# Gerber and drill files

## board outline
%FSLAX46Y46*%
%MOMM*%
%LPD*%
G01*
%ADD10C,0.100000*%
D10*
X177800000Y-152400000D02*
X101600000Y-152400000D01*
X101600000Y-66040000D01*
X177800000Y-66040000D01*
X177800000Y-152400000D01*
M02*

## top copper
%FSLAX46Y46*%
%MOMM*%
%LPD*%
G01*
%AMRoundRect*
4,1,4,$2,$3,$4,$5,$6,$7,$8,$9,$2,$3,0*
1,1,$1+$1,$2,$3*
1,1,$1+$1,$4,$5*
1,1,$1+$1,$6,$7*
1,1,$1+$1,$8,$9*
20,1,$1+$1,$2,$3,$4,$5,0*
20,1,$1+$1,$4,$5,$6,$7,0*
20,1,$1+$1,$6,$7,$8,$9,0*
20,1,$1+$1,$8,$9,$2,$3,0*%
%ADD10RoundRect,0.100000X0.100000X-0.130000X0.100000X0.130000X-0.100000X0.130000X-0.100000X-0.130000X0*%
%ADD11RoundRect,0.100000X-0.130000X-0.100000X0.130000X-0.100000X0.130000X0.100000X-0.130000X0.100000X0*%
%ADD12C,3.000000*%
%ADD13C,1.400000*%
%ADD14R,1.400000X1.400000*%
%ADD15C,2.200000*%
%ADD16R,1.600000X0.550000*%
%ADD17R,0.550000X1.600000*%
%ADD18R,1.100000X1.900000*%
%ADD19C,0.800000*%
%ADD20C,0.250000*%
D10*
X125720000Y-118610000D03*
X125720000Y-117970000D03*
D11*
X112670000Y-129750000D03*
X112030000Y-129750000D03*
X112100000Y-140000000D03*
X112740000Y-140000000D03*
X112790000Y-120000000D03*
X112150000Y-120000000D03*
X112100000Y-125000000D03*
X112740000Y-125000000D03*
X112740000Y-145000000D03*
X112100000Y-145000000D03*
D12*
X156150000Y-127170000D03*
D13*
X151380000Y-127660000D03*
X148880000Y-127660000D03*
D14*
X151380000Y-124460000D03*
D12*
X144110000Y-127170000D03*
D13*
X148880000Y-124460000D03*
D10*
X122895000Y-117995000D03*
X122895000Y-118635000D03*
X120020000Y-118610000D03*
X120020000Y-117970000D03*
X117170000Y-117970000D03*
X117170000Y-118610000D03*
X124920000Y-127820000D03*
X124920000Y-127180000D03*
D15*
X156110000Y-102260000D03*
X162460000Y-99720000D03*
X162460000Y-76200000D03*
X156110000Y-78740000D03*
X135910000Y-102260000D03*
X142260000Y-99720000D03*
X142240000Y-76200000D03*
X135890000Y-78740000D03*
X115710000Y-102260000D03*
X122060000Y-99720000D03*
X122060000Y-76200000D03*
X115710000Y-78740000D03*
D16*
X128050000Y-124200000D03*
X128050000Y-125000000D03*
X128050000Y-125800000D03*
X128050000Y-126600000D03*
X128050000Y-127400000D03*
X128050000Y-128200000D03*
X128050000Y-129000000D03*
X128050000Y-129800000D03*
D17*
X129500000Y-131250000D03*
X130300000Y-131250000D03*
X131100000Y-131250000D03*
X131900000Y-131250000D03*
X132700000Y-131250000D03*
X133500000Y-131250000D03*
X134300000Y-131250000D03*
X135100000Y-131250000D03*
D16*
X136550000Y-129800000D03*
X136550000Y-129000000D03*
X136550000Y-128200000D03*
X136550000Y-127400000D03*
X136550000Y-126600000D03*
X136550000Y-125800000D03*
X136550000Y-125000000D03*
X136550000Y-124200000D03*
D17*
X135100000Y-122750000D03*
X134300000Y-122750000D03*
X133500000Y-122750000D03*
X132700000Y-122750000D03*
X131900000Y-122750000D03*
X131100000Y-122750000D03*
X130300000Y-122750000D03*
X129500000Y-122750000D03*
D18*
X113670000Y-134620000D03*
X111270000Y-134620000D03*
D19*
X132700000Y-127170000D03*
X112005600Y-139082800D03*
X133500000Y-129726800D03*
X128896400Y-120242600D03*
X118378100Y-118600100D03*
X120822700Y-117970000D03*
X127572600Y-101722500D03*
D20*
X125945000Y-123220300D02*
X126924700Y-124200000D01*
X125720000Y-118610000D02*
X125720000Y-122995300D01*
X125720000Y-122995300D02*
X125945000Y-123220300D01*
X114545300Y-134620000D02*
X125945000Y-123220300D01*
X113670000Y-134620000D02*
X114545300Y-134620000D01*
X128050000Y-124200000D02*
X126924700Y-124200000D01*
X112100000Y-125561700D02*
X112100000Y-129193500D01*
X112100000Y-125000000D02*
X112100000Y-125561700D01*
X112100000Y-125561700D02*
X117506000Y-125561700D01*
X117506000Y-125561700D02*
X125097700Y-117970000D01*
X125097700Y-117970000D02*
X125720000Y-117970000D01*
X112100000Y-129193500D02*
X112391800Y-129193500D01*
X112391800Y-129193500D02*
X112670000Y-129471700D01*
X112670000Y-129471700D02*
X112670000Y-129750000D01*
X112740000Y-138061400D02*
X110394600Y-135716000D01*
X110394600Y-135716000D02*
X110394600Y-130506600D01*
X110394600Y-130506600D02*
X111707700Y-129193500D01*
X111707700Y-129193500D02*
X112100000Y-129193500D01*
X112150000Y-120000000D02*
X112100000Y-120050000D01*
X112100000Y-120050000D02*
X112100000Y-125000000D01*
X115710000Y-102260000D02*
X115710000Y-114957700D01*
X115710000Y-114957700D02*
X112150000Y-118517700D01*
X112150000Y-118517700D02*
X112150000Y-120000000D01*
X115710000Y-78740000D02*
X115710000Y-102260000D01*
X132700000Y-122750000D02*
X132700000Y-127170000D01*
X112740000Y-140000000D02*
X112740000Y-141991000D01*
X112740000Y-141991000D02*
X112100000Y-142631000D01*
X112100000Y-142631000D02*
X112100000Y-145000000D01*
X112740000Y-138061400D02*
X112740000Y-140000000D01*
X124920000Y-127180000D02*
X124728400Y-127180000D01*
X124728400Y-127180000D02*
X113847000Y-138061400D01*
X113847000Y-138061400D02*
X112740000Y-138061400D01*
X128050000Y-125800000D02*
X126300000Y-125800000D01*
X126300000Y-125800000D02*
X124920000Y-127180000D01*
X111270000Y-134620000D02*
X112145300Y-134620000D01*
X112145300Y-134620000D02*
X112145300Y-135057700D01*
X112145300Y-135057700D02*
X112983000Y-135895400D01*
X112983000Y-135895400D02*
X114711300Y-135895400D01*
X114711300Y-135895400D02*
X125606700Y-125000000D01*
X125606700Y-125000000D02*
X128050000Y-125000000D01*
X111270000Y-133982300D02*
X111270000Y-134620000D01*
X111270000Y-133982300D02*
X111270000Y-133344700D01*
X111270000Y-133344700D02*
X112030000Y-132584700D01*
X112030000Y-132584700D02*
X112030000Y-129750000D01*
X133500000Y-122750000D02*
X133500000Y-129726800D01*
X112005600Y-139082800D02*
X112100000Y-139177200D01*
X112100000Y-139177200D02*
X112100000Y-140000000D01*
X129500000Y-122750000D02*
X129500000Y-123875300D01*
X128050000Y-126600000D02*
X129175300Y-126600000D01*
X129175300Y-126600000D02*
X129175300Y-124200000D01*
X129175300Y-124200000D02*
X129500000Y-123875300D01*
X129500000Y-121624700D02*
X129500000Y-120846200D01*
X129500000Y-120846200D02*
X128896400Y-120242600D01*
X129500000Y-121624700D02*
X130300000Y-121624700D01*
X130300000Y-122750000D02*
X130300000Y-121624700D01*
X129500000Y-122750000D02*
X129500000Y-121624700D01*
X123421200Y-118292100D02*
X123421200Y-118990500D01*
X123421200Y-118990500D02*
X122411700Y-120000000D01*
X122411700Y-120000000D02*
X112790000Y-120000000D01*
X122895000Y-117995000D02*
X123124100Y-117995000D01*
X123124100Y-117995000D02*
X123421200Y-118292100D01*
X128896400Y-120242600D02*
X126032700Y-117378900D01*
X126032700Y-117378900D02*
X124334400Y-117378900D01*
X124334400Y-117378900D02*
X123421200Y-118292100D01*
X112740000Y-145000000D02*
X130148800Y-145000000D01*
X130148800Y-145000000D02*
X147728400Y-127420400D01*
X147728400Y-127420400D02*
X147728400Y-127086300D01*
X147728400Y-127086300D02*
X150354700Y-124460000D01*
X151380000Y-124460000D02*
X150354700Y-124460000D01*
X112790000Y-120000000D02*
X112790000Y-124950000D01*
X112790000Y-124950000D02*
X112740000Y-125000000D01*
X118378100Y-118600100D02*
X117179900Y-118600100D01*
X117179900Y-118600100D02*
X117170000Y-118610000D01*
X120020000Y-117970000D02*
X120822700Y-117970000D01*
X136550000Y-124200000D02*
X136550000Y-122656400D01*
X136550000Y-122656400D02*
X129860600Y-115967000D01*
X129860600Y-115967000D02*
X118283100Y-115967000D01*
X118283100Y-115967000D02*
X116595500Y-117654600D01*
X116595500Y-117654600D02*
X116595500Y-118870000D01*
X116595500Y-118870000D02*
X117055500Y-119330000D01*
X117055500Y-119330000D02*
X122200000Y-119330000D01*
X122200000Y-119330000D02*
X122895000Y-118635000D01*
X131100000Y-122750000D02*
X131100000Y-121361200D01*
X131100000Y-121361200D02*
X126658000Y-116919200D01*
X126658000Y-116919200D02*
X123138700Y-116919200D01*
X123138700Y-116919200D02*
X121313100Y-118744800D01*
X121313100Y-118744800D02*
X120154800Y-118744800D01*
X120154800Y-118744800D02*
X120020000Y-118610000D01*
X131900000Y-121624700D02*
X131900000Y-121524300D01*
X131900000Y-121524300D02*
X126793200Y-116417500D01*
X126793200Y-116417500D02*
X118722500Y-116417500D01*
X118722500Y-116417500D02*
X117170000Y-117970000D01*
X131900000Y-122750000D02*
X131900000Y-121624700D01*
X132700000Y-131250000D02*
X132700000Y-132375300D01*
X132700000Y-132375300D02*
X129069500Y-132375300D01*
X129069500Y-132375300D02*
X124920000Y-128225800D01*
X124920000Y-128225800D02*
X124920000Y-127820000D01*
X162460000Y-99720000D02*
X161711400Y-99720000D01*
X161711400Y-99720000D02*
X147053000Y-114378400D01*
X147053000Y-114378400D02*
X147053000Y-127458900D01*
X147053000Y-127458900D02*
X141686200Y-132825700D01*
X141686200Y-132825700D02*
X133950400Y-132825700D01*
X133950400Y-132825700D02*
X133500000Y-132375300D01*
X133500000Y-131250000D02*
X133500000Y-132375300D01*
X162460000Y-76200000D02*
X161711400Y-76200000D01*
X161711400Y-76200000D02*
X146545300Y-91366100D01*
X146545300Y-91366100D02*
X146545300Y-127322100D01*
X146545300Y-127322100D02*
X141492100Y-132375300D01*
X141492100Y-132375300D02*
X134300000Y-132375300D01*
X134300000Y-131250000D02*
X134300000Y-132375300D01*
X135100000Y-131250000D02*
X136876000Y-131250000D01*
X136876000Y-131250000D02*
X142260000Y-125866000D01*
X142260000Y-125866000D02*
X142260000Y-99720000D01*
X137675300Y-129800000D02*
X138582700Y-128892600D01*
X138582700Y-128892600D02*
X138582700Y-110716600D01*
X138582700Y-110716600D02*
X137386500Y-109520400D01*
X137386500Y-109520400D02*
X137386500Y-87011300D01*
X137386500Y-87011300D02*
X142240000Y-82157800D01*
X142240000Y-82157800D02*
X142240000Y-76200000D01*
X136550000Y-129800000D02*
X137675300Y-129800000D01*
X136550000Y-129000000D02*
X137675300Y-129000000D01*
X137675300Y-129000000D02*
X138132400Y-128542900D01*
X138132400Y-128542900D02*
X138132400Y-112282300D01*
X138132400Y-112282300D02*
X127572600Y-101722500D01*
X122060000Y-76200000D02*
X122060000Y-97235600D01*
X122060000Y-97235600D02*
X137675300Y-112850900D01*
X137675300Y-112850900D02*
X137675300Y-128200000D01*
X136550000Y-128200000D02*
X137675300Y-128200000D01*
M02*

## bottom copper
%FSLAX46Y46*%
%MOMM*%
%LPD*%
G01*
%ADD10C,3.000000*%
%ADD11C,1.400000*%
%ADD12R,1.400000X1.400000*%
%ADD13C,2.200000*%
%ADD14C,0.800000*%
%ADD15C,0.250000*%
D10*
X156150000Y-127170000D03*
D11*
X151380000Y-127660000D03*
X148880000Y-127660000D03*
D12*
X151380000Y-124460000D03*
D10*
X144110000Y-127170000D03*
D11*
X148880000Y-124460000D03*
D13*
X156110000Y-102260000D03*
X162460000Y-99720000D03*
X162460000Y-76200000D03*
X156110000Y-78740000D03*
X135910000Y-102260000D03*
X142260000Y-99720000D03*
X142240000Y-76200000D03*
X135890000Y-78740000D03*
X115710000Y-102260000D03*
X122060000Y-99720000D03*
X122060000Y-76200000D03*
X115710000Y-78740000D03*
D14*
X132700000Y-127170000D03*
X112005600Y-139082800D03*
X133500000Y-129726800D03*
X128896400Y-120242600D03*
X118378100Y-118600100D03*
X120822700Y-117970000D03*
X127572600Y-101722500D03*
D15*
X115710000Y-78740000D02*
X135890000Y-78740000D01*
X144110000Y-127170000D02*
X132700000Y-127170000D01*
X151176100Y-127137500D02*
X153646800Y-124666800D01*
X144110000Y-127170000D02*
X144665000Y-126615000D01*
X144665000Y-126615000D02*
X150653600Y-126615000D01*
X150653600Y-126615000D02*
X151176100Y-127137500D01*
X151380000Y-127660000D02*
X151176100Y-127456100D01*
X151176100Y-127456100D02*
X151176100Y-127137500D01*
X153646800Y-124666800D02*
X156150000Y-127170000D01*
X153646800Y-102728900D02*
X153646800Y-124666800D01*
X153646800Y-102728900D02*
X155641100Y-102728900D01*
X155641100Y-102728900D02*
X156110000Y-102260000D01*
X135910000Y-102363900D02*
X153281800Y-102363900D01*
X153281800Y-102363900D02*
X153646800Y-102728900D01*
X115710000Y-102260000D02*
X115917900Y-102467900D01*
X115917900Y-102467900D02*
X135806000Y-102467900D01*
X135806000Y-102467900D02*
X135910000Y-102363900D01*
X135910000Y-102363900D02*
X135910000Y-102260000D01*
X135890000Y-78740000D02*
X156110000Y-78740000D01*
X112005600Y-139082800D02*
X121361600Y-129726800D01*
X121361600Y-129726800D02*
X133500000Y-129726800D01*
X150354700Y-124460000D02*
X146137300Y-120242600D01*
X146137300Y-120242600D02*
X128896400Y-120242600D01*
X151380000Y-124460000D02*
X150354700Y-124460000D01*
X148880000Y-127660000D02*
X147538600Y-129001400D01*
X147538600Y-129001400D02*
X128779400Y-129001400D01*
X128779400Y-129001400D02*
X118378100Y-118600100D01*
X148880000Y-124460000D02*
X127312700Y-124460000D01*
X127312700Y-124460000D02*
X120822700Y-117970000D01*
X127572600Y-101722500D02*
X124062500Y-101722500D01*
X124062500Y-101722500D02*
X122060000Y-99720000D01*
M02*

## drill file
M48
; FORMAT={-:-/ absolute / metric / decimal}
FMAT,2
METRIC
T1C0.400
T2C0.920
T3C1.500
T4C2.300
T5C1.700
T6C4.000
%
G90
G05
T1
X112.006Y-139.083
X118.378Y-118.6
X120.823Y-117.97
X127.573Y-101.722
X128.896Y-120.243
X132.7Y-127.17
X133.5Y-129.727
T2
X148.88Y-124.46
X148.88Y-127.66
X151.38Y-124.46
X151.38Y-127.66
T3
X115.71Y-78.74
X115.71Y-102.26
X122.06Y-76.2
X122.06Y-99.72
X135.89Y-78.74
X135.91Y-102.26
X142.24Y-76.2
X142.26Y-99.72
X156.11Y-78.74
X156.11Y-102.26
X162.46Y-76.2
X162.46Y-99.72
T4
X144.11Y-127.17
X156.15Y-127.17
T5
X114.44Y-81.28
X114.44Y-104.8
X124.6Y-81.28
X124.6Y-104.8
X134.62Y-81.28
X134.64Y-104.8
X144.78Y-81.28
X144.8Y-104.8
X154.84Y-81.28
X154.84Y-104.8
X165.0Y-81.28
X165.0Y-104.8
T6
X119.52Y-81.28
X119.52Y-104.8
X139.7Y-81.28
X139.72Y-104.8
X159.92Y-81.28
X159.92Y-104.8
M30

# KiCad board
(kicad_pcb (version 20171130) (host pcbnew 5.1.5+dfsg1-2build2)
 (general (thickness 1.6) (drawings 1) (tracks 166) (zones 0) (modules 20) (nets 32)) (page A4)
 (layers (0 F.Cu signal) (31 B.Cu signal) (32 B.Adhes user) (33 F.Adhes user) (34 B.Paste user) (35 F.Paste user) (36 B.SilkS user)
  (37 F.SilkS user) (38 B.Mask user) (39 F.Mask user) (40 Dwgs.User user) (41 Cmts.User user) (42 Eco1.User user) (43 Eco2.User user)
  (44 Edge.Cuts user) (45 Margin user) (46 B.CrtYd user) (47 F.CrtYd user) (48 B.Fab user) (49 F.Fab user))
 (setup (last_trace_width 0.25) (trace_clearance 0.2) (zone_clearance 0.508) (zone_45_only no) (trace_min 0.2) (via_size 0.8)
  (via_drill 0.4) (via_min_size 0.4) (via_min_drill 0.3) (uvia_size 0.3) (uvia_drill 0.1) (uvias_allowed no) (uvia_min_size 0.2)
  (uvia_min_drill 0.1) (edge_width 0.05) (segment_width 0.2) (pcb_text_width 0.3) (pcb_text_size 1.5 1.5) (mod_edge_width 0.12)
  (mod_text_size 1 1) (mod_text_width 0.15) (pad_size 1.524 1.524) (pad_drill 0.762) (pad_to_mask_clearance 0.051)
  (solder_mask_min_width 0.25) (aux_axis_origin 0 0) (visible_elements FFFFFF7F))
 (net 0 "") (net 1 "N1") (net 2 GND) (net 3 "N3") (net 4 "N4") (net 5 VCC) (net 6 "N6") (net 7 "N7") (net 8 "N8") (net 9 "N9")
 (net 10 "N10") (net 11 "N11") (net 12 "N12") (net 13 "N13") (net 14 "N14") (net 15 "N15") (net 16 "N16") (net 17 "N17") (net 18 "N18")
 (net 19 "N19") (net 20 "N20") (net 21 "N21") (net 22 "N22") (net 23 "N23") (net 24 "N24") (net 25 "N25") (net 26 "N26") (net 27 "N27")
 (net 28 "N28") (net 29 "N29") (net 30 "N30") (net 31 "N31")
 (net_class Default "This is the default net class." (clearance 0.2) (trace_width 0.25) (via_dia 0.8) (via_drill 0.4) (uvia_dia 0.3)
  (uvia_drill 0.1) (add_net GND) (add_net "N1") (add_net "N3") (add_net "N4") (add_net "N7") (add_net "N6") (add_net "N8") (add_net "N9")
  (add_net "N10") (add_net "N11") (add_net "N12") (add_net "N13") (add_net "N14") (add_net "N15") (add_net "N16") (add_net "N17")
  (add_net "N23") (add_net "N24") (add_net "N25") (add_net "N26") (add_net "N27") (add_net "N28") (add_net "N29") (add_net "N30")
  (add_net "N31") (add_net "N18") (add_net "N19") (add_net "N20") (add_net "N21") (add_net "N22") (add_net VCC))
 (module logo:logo (layer F.Cu) (at 149.86 141.5)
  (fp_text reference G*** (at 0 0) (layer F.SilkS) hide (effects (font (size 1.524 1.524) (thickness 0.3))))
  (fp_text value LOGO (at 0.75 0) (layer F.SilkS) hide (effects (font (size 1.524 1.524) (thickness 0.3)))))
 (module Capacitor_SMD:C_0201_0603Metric (layer F.Cu) (at 125.72 118.29 90)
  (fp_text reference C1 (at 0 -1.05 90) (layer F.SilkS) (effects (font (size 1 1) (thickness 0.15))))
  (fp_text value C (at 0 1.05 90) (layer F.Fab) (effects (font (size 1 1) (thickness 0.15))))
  (pad "" smd roundrect (at -0.345 0 90) (size 0.318 0.36) (layers F.Paste) (roundrect_rratio 0.25))
  (pad "" smd roundrect (at 0.345 0 90) (size 0.318 0.36) (layers F.Paste) (roundrect_rratio 0.25))
  (pad 1 smd roundrect (at -0.32 0 90) (size 0.46 0.4) (layers F.Cu F.Mask) (roundrect_rratio 0.25) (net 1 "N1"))
  (pad 2 smd roundrect (at 0.32 0 90) (size 0.46 0.4) (layers F.Cu F.Mask) (roundrect_rratio 0.25) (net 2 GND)))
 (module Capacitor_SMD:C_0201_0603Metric (layer F.Cu) (at 112.35 129.75)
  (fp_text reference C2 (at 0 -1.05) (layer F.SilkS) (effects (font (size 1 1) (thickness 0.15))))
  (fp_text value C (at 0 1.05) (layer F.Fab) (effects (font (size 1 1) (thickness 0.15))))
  (pad 2 smd roundrect (at 0.32 0) (size 0.46 0.4) (layers F.Cu F.Mask) (roundrect_rratio 0.25) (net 2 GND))
  (pad 1 smd roundrect (at -0.32 0) (size 0.46 0.4) (layers F.Cu F.Mask) (roundrect_rratio 0.25) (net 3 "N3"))
  (pad "" smd roundrect (at 0.345 0) (size 0.318 0.36) (layers F.Paste) (roundrect_rratio 0.25))
  (pad "" smd roundrect (at -0.345 0) (size 0.318 0.36) (layers F.Paste) (roundrect_rratio 0.25)))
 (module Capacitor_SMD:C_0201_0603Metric (layer F.Cu) (at 112.42 140)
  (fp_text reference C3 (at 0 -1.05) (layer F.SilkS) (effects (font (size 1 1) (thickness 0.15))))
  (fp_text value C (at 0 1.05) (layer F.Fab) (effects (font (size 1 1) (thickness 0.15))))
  (pad "" smd roundrect (at -0.345 0) (size 0.318 0.36) (layers F.Paste) (roundrect_rratio 0.25))
  (pad "" smd roundrect (at 0.345 0) (size 0.318 0.36) (layers F.Paste) (roundrect_rratio 0.25))
  (pad 1 smd roundrect (at -0.32 0) (size 0.46 0.4) (layers F.Cu F.Mask) (roundrect_rratio 0.25) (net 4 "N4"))
  (pad 2 smd roundrect (at 0.32 0) (size 0.46 0.4) (layers F.Cu F.Mask) (roundrect_rratio 0.25) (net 2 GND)))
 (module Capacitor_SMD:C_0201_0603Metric (layer F.Cu) (at 112.47 120)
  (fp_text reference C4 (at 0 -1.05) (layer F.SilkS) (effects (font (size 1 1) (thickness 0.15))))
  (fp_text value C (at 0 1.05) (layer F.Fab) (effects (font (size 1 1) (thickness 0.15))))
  (pad 2 smd roundrect (at 0.32 0) (size 0.46 0.4) (layers F.Cu F.Mask) (roundrect_rratio 0.25) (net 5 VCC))
  (pad 1 smd roundrect (at -0.32 0) (size 0.46 0.4) (layers F.Cu F.Mask) (roundrect_rratio 0.25) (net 2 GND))
  (pad "" smd roundrect (at 0.345 0) (size 0.318 0.36) (layers F.Paste) (roundrect_rratio 0.25))
  (pad "" smd roundrect (at -0.345 0) (size 0.318 0.36) (layers F.Paste) (roundrect_rratio 0.25)))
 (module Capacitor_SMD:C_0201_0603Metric (layer F.Cu) (at 112.42 125)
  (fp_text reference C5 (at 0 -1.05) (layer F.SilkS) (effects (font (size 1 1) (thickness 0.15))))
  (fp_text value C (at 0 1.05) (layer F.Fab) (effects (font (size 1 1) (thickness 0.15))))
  (pad "" smd roundrect (at -0.345 0) (size 0.318 0.36) (layers F.Paste) (roundrect_rratio 0.25))
  (pad "" smd roundrect (at 0.345 0) (size 0.318 0.36) (layers F.Paste) (roundrect_rratio 0.25))
  (pad 1 smd roundrect (at -0.32 0) (size 0.46 0.4) (layers F.Cu F.Mask) (roundrect_rratio 0.25) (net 2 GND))
  (pad 2 smd roundrect (at 0.32 0) (size 0.46 0.4) (layers F.Cu F.Mask) (roundrect_rratio 0.25) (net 5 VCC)))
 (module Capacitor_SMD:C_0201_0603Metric (layer F.Cu) (at 112.42 145)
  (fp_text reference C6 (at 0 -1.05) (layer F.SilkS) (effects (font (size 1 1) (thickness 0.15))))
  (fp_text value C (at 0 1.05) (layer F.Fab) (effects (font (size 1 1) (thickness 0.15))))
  (pad 2 smd roundrect (at 0.32 0) (size 0.46 0.4) (layers F.Cu F.Mask) (roundrect_rratio 0.25) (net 5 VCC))
  (pad 1 smd roundrect (at -0.32 0) (size 0.46 0.4) (layers F.Cu F.Mask) (roundrect_rratio 0.25) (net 2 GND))
  (pad "" smd roundrect (at 0.345 0) (size 0.318 0.36) (layers F.Paste) (roundrect_rratio 0.25))
  (pad "" smd roundrect (at -0.345 0) (size 0.318 0.36) (layers F.Paste) (roundrect_rratio 0.25)))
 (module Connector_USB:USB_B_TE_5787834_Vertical (layer F.Cu) (at 151.38 124.46)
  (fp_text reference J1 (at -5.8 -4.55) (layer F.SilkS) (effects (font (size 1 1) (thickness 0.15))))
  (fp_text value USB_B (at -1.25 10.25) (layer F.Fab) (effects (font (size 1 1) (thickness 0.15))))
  (pad 5 thru_hole circle (at 4.77 2.71) (size 3 3) (drill 2.3) (layers *.Cu *.Mask) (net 2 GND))
  (pad 4 thru_hole circle (at 0 3.2) (size 1.4 1.4) (drill 0.92) (layers *.Cu *.Mask) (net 2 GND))
  (pad 3 thru_hole circle (at -2.5 3.2) (size 1.4 1.4) (drill 0.92) (layers *.Cu *.Mask) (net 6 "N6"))
  (pad 1 thru_hole rect (at 0 0) (size 1.4 1.4) (drill 0.92) (layers *.Cu *.Mask) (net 5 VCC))
  (pad 5 thru_hole circle (at -7.27 2.71) (size 3 3) (drill 2.3) (layers *.Cu *.Mask) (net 2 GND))
  (pad 2 thru_hole circle (at -2.5 0) (size 1.4 1.4) (drill 0.92) (layers *.Cu *.Mask) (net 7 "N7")))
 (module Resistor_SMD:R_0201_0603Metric (layer F.Cu) (at 122.895 118.315 90)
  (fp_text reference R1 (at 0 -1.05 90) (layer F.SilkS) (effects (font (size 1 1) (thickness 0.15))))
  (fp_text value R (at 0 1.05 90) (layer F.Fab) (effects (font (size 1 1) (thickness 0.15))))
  (pad 2 smd roundrect (at 0.32 0 90) (size 0.46 0.4) (layers F.Cu F.Mask) (roundrect_rratio 0.25) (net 5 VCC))
  (pad 1 smd roundrect (at -0.32 0 90) (size 0.46 0.4) (layers F.Cu F.Mask) (roundrect_rratio 0.25) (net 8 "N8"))
  (pad "" smd roundrect (at 0.345 0 90) (size 0.318 0.36) (layers F.Paste) (roundrect_rratio 0.25))
  (pad "" smd roundrect (at -0.345 0 90) (size 0.318 0.36) (layers F.Paste) (roundrect_rratio 0.25)))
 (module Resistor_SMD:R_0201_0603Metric (layer F.Cu) (at 120.02 118.29 90)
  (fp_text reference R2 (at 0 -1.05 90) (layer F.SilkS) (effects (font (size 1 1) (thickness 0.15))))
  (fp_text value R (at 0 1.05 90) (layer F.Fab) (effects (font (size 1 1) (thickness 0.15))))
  (pad "" smd roundrect (at -0.345 0 90) (size 0.318 0.36) (layers F.Paste) (roundrect_rratio 0.25))
  (pad "" smd roundrect (at 0.345 0 90) (size 0.318 0.36) (layers F.Paste) (roundrect_rratio 0.25))
  (pad 1 smd roundrect (at -0.32 0 90) (size 0.46 0.4) (layers F.Cu F.Mask) (roundrect_rratio 0.25) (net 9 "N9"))
  (pad 2 smd roundrect (at 0.32 0 90) (size 0.46 0.4) (layers F.Cu F.Mask) (roundrect_rratio 0.25) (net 7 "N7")))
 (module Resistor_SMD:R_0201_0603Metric (layer F.Cu) (at 117.17 118.29 90)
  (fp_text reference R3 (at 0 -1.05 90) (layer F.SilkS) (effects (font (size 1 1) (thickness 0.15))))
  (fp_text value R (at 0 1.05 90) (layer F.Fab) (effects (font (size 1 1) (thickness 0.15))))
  (pad 2 smd roundrect (at 0.32 0 90) (size 0.46 0.4) (layers F.Cu F.Mask) (roundrect_rratio 0.25) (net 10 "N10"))
  (pad 1 smd roundrect (at -0.32 0 90) (size 0.46 0.4) (layers F.Cu F.Mask) (roundrect_rratio 0.25) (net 6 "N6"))
  (pad "" smd roundrect (at 0.345 0 90) (size 0.318 0.36) (layers F.Paste) (roundrect_rratio 0.25))
  (pad "" smd roundrect (at -0.345 0 90) (size 0.318 0.36) (layers F.Paste) (roundrect_rratio 0.25)))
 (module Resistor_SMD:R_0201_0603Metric (layer F.Cu) (at 124.92 127.5 90)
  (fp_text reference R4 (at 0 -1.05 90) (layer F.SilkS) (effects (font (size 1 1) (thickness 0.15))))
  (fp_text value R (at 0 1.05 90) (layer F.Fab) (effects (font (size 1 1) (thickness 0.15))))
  (pad "" smd roundrect (at -0.345 0 90) (size 0.318 0.36) (layers F.Paste) (roundrect_rratio 0.25))
  (pad "" smd roundrect (at 0.345 0 90) (size 0.318 0.36) (layers F.Paste) (roundrect_rratio 0.25))
  (pad 1 smd roundrect (at -0.32 0 90) (size 0.46 0.4) (layers F.Cu F.Mask) (roundrect_rratio 0.25) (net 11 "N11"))
  (pad 2 smd roundrect (at 0.32 0 90) (size 0.46 0.4) (layers F.Cu F.Mask) (roundrect_rratio 0.25) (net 2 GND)))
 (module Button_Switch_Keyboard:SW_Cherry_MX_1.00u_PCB (layer F.Cu) (at 162.46 99.72)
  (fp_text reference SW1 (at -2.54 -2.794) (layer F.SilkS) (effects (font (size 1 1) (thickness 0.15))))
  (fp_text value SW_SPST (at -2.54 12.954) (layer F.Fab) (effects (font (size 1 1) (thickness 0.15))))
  (pad "" np_thru_hole circle (at 2.54 5.08) (size 1.7 1.7) (drill 1.7) (layers *.Cu *.Mask))
  (pad "" np_thru_hole circle (at -7.62 5.08) (size 1.7 1.7) (drill 1.7) (layers *.Cu *.Mask))
  (pad "" np_thru_hole circle (at -2.54 5.08) (size 4 4) (drill 4) (layers *.Cu *.Mask))
  (pad 2 thru_hole circle (at -6.35 2.54) (size 2.2 2.2) (drill 1.5) (layers *.Cu *.Mask) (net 2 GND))
  (pad 1 thru_hole circle (at 0 0) (size 2.2 2.2) (drill 1.5) (layers *.Cu *.Mask) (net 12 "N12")))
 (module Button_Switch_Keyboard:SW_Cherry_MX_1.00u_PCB (layer F.Cu) (at 162.46 76.2)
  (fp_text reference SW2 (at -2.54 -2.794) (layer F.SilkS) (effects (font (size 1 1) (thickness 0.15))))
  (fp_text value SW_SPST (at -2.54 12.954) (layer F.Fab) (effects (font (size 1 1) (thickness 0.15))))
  (pad 1 thru_hole circle (at 0 0) (size 2.2 2.2) (drill 1.5) (layers *.Cu *.Mask) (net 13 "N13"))
  (pad 2 thru_hole circle (at -6.35 2.54) (size 2.2 2.2) (drill 1.5) (layers *.Cu *.Mask) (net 2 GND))
  (pad "" np_thru_hole circle (at -2.54 5.08) (size 4 4) (drill 4) (layers *.Cu *.Mask))
  (pad "" np_thru_hole circle (at -7.62 5.08) (size 1.7 1.7) (drill 1.7) (layers *.Cu *.Mask))
  (pad "" np_thru_hole circle (at 2.54 5.08) (size 1.7 1.7) (drill 1.7) (layers *.Cu *.Mask)))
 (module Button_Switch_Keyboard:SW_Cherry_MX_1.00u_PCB (layer F.Cu) (at 142.26 99.72)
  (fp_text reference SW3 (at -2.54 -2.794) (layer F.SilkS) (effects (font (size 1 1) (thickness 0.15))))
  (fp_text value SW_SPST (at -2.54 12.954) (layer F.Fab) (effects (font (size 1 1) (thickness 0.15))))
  (pad "" np_thru_hole circle (at 2.54 5.08) (size 1.7 1.7) (drill 1.7) (layers *.Cu *.Mask))
  (pad "" np_thru_hole circle (at -7.62 5.08) (size 1.7 1.7) (drill 1.7) (layers *.Cu *.Mask))
  (pad "" np_thru_hole circle (at -2.54 5.08) (size 4 4) (drill 4) (layers *.Cu *.Mask))
  (pad 2 thru_hole circle (at -6.35 2.54) (size 2.2 2.2) (drill 1.5) (layers *.Cu *.Mask) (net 2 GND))
  (pad 1 thru_hole circle (at 0 0) (size 2.2 2.2) (drill 1.5) (layers *.Cu *.Mask) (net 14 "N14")))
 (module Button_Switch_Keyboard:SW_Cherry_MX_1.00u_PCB (layer F.Cu) (at 142.24 76.2)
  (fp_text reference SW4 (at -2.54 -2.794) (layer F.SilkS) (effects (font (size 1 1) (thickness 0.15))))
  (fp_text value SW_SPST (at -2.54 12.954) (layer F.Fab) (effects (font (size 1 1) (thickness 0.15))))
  (pad 1 thru_hole circle (at 0 0) (size 2.2 2.2) (drill 1.5) (layers *.Cu *.Mask) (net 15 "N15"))
  (pad 2 thru_hole circle (at -6.35 2.54) (size 2.2 2.2) (drill 1.5) (layers *.Cu *.Mask) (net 2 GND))
  (pad "" np_thru_hole circle (at -2.54 5.08) (size 4 4) (drill 4) (layers *.Cu *.Mask))
  (pad "" np_thru_hole circle (at -7.62 5.08) (size 1.7 1.7) (drill 1.7) (layers *.Cu *.Mask))
  (pad "" np_thru_hole circle (at 2.54 5.08) (size 1.7 1.7) (drill 1.7) (layers *.Cu *.Mask)))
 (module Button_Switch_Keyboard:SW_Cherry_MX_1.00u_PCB (layer F.Cu) (at 122.06 99.72)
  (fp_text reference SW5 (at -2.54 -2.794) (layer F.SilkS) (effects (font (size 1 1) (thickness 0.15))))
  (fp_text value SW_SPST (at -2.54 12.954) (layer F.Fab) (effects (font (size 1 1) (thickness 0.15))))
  (pad "" np_thru_hole circle (at 2.54 5.08) (size 1.7 1.7) (drill 1.7) (layers *.Cu *.Mask))
  (pad "" np_thru_hole circle (at -7.62 5.08) (size 1.7 1.7) (drill 1.7) (layers *.Cu *.Mask))
  (pad "" np_thru_hole circle (at -2.54 5.08) (size 4 4) (drill 4) (layers *.Cu *.Mask))
  (pad 2 thru_hole circle (at -6.35 2.54) (size 2.2 2.2) (drill 1.5) (layers *.Cu *.Mask) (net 2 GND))
  (pad 1 thru_hole circle (at 0 0) (size 2.2 2.2) (drill 1.5) (layers *.Cu *.Mask) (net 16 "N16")))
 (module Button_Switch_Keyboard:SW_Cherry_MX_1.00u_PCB (layer F.Cu) (at 122.06 76.2)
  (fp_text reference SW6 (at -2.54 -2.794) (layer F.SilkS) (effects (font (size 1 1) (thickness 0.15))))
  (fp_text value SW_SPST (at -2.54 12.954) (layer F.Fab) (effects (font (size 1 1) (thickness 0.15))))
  (pad 1 thru_hole circle (at 0 0) (size 2.2 2.2) (drill 1.5) (layers *.Cu *.Mask) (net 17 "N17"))
  (pad 2 thru_hole circle (at -6.35 2.54) (size 2.2 2.2) (drill 1.5) (layers *.Cu *.Mask) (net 2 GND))
  (pad "" np_thru_hole circle (at -2.54 5.08) (size 4 4) (drill 4) (layers *.Cu *.Mask))
  (pad "" np_thru_hole circle (at -7.62 5.08) (size 1.7 1.7) (drill 1.7) (layers *.Cu *.Mask))
  (pad "" np_thru_hole circle (at 2.54 5.08) (size 1.7 1.7) (drill 1.7) (layers *.Cu *.Mask)))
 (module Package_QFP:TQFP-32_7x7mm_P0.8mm (layer F.Cu) (at 132.3 127)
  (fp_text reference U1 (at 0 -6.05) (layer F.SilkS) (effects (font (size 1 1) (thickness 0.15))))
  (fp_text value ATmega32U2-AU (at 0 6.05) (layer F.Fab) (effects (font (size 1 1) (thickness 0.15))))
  (pad 1 smd rect (at -4.25 -2.8) (size 1.6 0.55) (layers F.Cu F.Paste F.Mask) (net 1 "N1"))
  (pad 2 smd rect (at -4.25 -2) (size 1.6 0.55) (layers F.Cu F.Paste F.Mask) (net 3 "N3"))
  (pad 3 smd rect (at -4.25 -1.2) (size 1.6 0.55) (layers F.Cu F.Paste F.Mask) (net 2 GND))
  (pad 4 smd rect (at -4.25 -0.4) (size 1.6 0.55) (layers F.Cu F.Paste F.Mask) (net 5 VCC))
  (pad 5 smd rect (at -4.25 0.4) (size 1.6 0.55) (layers F.Cu F.Paste F.Mask) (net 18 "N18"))
  (pad 6 smd rect (at -4.25 1.2) (size 1.6 0.55) (layers F.Cu F.Paste F.Mask) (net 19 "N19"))
  (pad 7 smd rect (at -4.25 2) (size 1.6 0.55) (layers F.Cu F.Paste F.Mask) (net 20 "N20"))
  (pad 8 smd rect (at -4.25 2.8) (size 1.6 0.55) (layers F.Cu F.Paste F.Mask) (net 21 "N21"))
  (pad 9 smd rect (at -2.8 4.25 90) (size 1.6 0.55) (layers F.Cu F.Paste F.Mask) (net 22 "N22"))
  (pad 10 smd rect (at -2 4.25 90) (size 1.6 0.55) (layers F.Cu F.Paste F.Mask) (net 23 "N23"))
  (pad 11 smd rect (at -1.2 4.25 90) (size 1.6 0.55) (layers F.Cu F.Paste F.Mask) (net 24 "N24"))
  (pad 12 smd rect (at -0.4 4.25 90) (size 1.6 0.55) (layers F.Cu F.Paste F.Mask) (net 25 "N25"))
  (pad 13 smd rect (at 0.4 4.25 90) (size 1.6 0.55) (layers F.Cu F.Paste F.Mask) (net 11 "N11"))
  (pad 14 smd rect (at 1.2 4.25 90) (size 1.6 0.55) (layers F.Cu F.Paste F.Mask) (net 12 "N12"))
  (pad 15 smd rect (at 2 4.25 90) (size 1.6 0.55) (layers F.Cu F.Paste F.Mask) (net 13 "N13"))
  (pad 16 smd rect (at 2.8 4.25 90) (size 1.6 0.55) (layers F.Cu F.Paste F.Mask) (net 14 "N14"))
  (pad 17 smd rect (at 4.25 2.8) (size 1.6 0.55) (layers F.Cu F.Paste F.Mask) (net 15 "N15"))
  (pad 18 smd rect (at 4.25 2) (size 1.6 0.55) (layers F.Cu F.Paste F.Mask) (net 16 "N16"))
  (pad 19 smd rect (at 4.25 1.2) (size 1.6 0.55) (layers F.Cu F.Paste F.Mask) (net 17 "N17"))
  (pad 20 smd rect (at 4.25 0.4) (size 1.6 0.55) (layers F.Cu F.Paste F.Mask) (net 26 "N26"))
  (pad 21 smd rect (at 4.25 -0.4) (size 1.6 0.55) (layers F.Cu F.Paste F.Mask) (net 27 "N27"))
  (pad 22 smd rect (at 4.25 -1.2) (size 1.6 0.55) (layers F.Cu F.Paste F.Mask) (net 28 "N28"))
  (pad 23 smd rect (at 4.25 -2) (size 1.6 0.55) (layers F.Cu F.Paste F.Mask) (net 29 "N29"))
  (pad 24 smd rect (at 4.25 -2.8) (size 1.6 0.55) (layers F.Cu F.Paste F.Mask) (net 8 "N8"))
  (pad 25 smd rect (at 2.8 -4.25 90) (size 1.6 0.55) (layers F.Cu F.Paste F.Mask) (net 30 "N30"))
  (pad 26 smd rect (at 2 -4.25 90) (size 1.6 0.55) (layers F.Cu F.Paste F.Mask) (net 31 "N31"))
  (pad 27 smd rect (at 1.2 -4.25 90) (size 1.6 0.55) (layers F.Cu F.Paste F.Mask) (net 4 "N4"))
  (pad 28 smd rect (at 0.4 -4.25 90) (size 1.6 0.55) (layers F.Cu F.Paste F.Mask) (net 2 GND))
  (pad 29 smd rect (at -0.4 -4.25 90) (size 1.6 0.55) (layers F.Cu F.Paste F.Mask) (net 10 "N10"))
  (pad 30 smd rect (at -1.2 -4.25 90) (size 1.6 0.55) (layers F.Cu F.Paste F.Mask) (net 9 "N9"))
  (pad 31 smd rect (at -2 -4.25 90) (size 1.6 0.55) (layers F.Cu F.Paste F.Mask) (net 5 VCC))
  (pad 32 smd rect (at -2.8 -4.25 90) (size 1.6 0.55) (layers F.Cu F.Paste F.Mask) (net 5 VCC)))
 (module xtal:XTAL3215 (layer F.Cu) (at 112.47 134.62)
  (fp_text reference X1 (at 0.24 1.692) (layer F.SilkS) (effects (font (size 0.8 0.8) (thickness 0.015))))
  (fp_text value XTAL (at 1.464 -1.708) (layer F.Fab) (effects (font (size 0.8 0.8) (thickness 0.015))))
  (pad P$1 smd rect (at 1.2 0) (size 1.1 1.9) (layers F.Cu F.Paste F.Mask) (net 1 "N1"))
  (pad P$2 smd rect (at -1.2 0) (size 1.1 1.9) (layers F.Cu F.Paste F.Mask) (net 3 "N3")))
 (gr_poly (pts (xy 177.8 152.4) (xy 101.6 152.4) (xy 101.6 66.04) (xy 177.8 66.04)) (layer Edge.Cuts) (width 0.1))
 (segment (start 125.945 123.2203) (end 126.9247 124.2) (width 0.25) (layer F.Cu) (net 1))
 (segment (start 125.72 118.61) (end 125.72 122.9953) (width 0.25) (layer F.Cu) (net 1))
 (segment (start 125.72 122.9953) (end 125.945 123.2203) (width 0.25) (layer F.Cu) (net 1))
 (segment (start 114.5453 134.62) (end 125.945 123.2203) (width 0.25) (layer F.Cu) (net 1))
 (segment (start 113.67 134.62) (end 114.5453 134.62) (width 0.25) (layer F.Cu) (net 1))
 (segment (start 128.05 124.2) (end 126.9247 124.2) (width 0.25) (layer F.Cu) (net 1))
 (segment (start 112.1 125.5617) (end 112.1 129.1935) (width 0.25) (layer F.Cu) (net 2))
 (segment (start 112.1 125) (end 112.1 125.5617) (width 0.25) (layer F.Cu) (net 2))
 (segment (start 112.1 125.5617) (end 117.506 125.5617) (width 0.25) (layer F.Cu) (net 2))
 (segment (start 117.506 125.5617) (end 125.0977 117.97) (width 0.25) (layer F.Cu) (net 2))
 (segment (start 125.0977 117.97) (end 125.72 117.97) (width 0.25) (layer F.Cu) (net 2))
 (segment (start 112.1 129.1935) (end 112.3918 129.1935) (width 0.25) (layer F.Cu) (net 2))
 (segment (start 112.3918 129.1935) (end 112.67 129.4717) (width 0.25) (layer F.Cu) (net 2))
 (segment (start 112.67 129.4717) (end 112.67 129.75) (width 0.25) (layer F.Cu) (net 2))
 (segment (start 112.74 138.0614) (end 110.3946 135.716) (width 0.25) (layer F.Cu) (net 2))
 (segment (start 110.3946 135.716) (end 110.3946 130.5066) (width 0.25) (layer F.Cu) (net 2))
 (segment (start 110.3946 130.5066) (end 111.7077 129.1935) (width 0.25) (layer F.Cu) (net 2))
 (segment (start 111.7077 129.1935) (end 112.1 129.1935) (width 0.25) (layer F.Cu) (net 2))
 (segment (start 112.15 120) (end 112.1 120.05) (width 0.25) (layer F.Cu) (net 2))
 (segment (start 112.1 120.05) (end 112.1 125) (width 0.25) (layer F.Cu) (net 2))
 (segment (start 115.71 102.26) (end 115.71 114.9577) (width 0.25) (layer F.Cu) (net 2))
 (segment (start 115.71 114.9577) (end 112.15 118.5177) (width 0.25) (layer F.Cu) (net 2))
 (segment (start 112.15 118.5177) (end 112.15 120) (width 0.25) (layer F.Cu) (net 2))
 (segment (start 115.71 78.74) (end 115.71 102.26) (width 0.25) (layer F.Cu) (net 2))
 (segment (start 132.7 122.75) (end 132.7 127.17) (width 0.25) (layer F.Cu) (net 2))
 (segment (start 115.71 78.74) (end 135.89 78.74) (width 0.25) (layer B.Cu) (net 2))
 (segment (start 144.11 127.17) (end 132.7 127.17) (width 0.25) (layer B.Cu) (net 2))
 (segment (start 112.74 140) (end 112.74 141.991) (width 0.25) (layer F.Cu) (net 2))
 (segment (start 112.74 141.991) (end 112.1 142.631) (width 0.25) (layer F.Cu) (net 2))
 (segment (start 112.1 142.631) (end 112.1 145) (width 0.25) (layer F.Cu) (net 2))
 (segment (start 112.74 138.0614) (end 112.74 140) (width 0.25) (layer F.Cu) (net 2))
 (segment (start 151.1761 127.1375) (end 153.6468 124.6668) (width 0.25) (layer B.Cu) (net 2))
 (segment (start 144.11 127.17) (end 144.665 126.615) (width 0.25) (layer B.Cu) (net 2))
 (segment (start 144.665 126.615) (end 150.6536 126.615) (width 0.25) (layer B.Cu) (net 2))
 (segment (start 150.6536 126.615) (end 151.1761 127.1375) (width 0.25) (layer B.Cu) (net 2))
 (segment (start 151.38 127.66) (end 151.1761 127.4561) (width 0.25) (layer B.Cu) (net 2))
 (segment (start 151.1761 127.4561) (end 151.1761 127.1375) (width 0.25) (layer B.Cu) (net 2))
 (segment (start 153.6468 124.6668) (end 156.15 127.17) (width 0.25) (layer B.Cu) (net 2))
 (segment (start 153.6468 102.7289) (end 153.6468 124.6668) (width 0.25) (layer B.Cu) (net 2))
 (segment (start 153.6468 102.7289) (end 155.6411 102.7289) (width 0.25) (layer B.Cu) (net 2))
 (segment (start 155.6411 102.7289) (end 156.11 102.26) (width 0.25) (layer B.Cu) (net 2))
 (segment (start 135.91 102.3639) (end 153.2818 102.3639) (width 0.25) (layer B.Cu) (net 2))
 (segment (start 153.2818 102.3639) (end 153.6468 102.7289) (width 0.25) (layer B.Cu) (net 2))
 (segment (start 124.92 127.18) (end 124.7284 127.18) (width 0.25) (layer F.Cu) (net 2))
 (segment (start 124.7284 127.18) (end 113.847 138.0614) (width 0.25) (layer F.Cu) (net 2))
 (segment (start 113.847 138.0614) (end 112.74 138.0614) (width 0.25) (layer F.Cu) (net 2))
 (segment (start 128.05 125.8) (end 126.3 125.8) (width 0.25) (layer F.Cu) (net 2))
 (segment (start 126.3 125.8) (end 124.92 127.18) (width 0.25) (layer F.Cu) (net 2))
 (segment (start 115.71 102.26) (end 115.9179 102.4679) (width 0.25) (layer B.Cu) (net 2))
 (segment (start 115.9179 102.4679) (end 135.806 102.4679) (width 0.25) (layer B.Cu) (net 2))
 (segment (start 135.806 102.4679) (end 135.91 102.3639) (width 0.25) (layer B.Cu) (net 2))
 (segment (start 135.91 102.3639) (end 135.91 102.26) (width 0.25) (layer B.Cu) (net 2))
 (segment (start 135.89 78.74) (end 156.11 78.74) (width 0.25) (layer B.Cu) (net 2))
 (via (at 132.7 127.17) (size 0.8) (layers F.Cu B.Cu) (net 2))
 (segment (start 111.27 134.62) (end 112.1453 134.62) (width 0.25) (layer F.Cu) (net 3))
 (segment (start 112.1453 134.62) (end 112.1453 135.0577) (width 0.25) (layer F.Cu) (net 3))
 (segment (start 112.1453 135.0577) (end 112.983 135.8954) (width 0.25) (layer F.Cu) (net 3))
 (segment (start 112.983 135.8954) (end 114.7113 135.8954) (width 0.25) (layer F.Cu) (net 3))
 (segment (start 114.7113 135.8954) (end 125.6067 125) (width 0.25) (layer F.Cu) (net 3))
 (segment (start 125.6067 125) (end 128.05 125) (width 0.25) (layer F.Cu) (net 3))
 (segment (start 111.27 133.9823) (end 111.27 134.62) (width 0.25) (layer F.Cu) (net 3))
 (segment (start 111.27 133.9823) (end 111.27 133.3447) (width 0.25) (layer F.Cu) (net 3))
 (segment (start 111.27 133.3447) (end 112.03 132.5847) (width 0.25) (layer F.Cu) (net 3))
 (segment (start 112.03 132.5847) (end 112.03 129.75) (width 0.25) (layer F.Cu) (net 3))
 (segment (start 133.5 122.75) (end 133.5 129.7268) (width 0.25) (layer F.Cu) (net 4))
 (segment (start 112.0056 139.0828) (end 121.3616 129.7268) (width 0.25) (layer B.Cu) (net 4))
 (segment (start 121.3616 129.7268) (end 133.5 129.7268) (width 0.25) (layer B.Cu) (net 4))
 (segment (start 112.0056 139.0828) (end 112.1 139.1772) (width 0.25) (layer F.Cu) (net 4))
 (segment (start 112.1 139.1772) (end 112.1 140) (width 0.25) (layer F.Cu) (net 4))
 (via (at 112.0056 139.0828) (size 0.8) (layers F.Cu B.Cu) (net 4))
 (via (at 133.5 129.7268) (size 0.8) (layers F.Cu B.Cu) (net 4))
 (segment (start 129.5 122.75) (end 129.5 123.8753) (width 0.25) (layer F.Cu) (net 5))
 (segment (start 128.05 126.6) (end 129.1753 126.6) (width 0.25) (layer F.Cu) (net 5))
 (segment (start 129.1753 126.6) (end 129.1753 124.2) (width 0.25) (layer F.Cu) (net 5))
 (segment (start 129.1753 124.2) (end 129.5 123.8753) (width 0.25) (layer F.Cu) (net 5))
 (segment (start 129.5 121.6247) (end 129.5 120.8462) (width 0.25) (layer F.Cu) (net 5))
 (segment (start 129.5 120.8462) (end 128.8964 120.2426) (width 0.25) (layer F.Cu) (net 5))
 (segment (start 129.5 121.6247) (end 130.3 121.6247) (width 0.25) (layer F.Cu) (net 5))
 (segment (start 130.3 122.75) (end 130.3 121.6247) (width 0.25) (layer F.Cu) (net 5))
 (segment (start 129.5 122.75) (end 129.5 121.6247) (width 0.25) (layer F.Cu) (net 5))
 (segment (start 123.4212 118.2921) (end 123.4212 118.9905) (width 0.25) (layer F.Cu) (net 5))
 (segment (start 123.4212 118.9905) (end 122.4117 120) (width 0.25) (layer F.Cu) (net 5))
 (segment (start 122.4117 120) (end 112.79 120) (width 0.25) (layer F.Cu) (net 5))
 (segment (start 122.895 117.995) (end 123.1241 117.995) (width 0.25) (layer F.Cu) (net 5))
 (segment (start 123.1241 117.995) (end 123.4212 118.2921) (width 0.25) (layer F.Cu) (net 5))
 (segment (start 128.8964 120.2426) (end 126.0327 117.3789) (width 0.25) (layer F.Cu) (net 5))
 (segment (start 126.0327 117.3789) (end 124.3344 117.3789) (width 0.25) (layer F.Cu) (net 5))
 (segment (start 124.3344 117.3789) (end 123.4212 118.2921) (width 0.25) (layer F.Cu) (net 5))
 (segment (start 150.3547 124.46) (end 146.1373 120.2426) (width 0.25) (layer B.Cu) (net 5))
 (segment (start 146.1373 120.2426) (end 128.8964 120.2426) (width 0.25) (layer B.Cu) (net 5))
 (segment (start 151.38 124.46) (end 150.3547 124.46) (width 0.25) (layer B.Cu) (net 5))
 (segment (start 112.74 145) (end 130.1488 145) (width 0.25) (layer F.Cu) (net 5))
 (segment (start 130.1488 145) (end 147.7284 127.4204) (width 0.25) (layer F.Cu) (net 5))
 (segment (start 147.7284 127.4204) (end 147.7284 127.0863) (width 0.25) (layer F.Cu) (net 5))
 (segment (start 147.7284 127.0863) (end 150.3547 124.46) (width 0.25) (layer F.Cu) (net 5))
 (segment (start 151.38 124.46) (end 150.3547 124.46) (width 0.25) (layer F.Cu) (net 5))
 (segment (start 112.79 120) (end 112.79 124.95) (width 0.25) (layer F.Cu) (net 5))
 (segment (start 112.79 124.95) (end 112.74 125) (width 0.25) (layer F.Cu) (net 5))
 (via (at 128.8964 120.2426) (size 0.8) (layers F.Cu B.Cu) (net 5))
 (segment (start 118.3781 118.6001) (end 117.1799 118.6001) (width 0.25) (layer F.Cu) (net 6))
 (segment (start 117.1799 118.6001) (end 117.17 118.61) (width 0.25) (layer F.Cu) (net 6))
 (segment (start 148.88 127.66) (end 147.5386 129.0014) (width 0.25) (layer B.Cu) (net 6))
 (segment (start 147.5386 129.0014) (end 128.7794 129.0014) (width 0.25) (layer B.Cu) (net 6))
 (segment (start 128.7794 129.0014) (end 118.3781 118.6001) (width 0.25) (layer B.Cu) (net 6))
 (via (at 118.3781 118.6001) (size 0.8) (layers F.Cu B.Cu) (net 6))
 (segment (start 148.88 124.46) (end 127.3127 124.46) (width 0.25) (layer B.Cu) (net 7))
 (segment (start 127.3127 124.46) (end 120.8227 117.97) (width 0.25) (layer B.Cu) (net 7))
 (segment (start 120.02 117.97) (end 120.8227 117.97) (width 0.25) (layer F.Cu) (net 7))
 (via (at 120.8227 117.97) (size 0.8) (layers F.Cu B.Cu) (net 7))
 (segment (start 136.55 124.2) (end 136.55 122.6564) (width 0.25) (layer F.Cu) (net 8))
 (segment (start 136.55 122.6564) (end 129.8606 115.967) (width 0.25) (layer F.Cu) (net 8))
 (segment (start 129.8606 115.967) (end 118.2831 115.967) (width 0.25) (layer F.Cu) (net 8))
 (segment (start 118.2831 115.967) (end 116.5955 117.6546) (width 0.25) (layer F.Cu) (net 8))
 (segment (start 116.5955 117.6546) (end 116.5955 118.87) (width 0.25) (layer F.Cu) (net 8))
 (segment (start 116.5955 118.87) (end 117.0555 119.33) (width 0.25) (layer F.Cu) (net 8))
 (segment (start 117.0555 119.33) (end 122.2 119.33) (width 0.25) (layer F.Cu) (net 8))
 (segment (start 122.2 119.33) (end 122.895 118.635) (width 0.25) (layer F.Cu) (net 8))
 (segment (start 131.1 122.75) (end 131.1 121.3612) (width 0.25) (layer F.Cu) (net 9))
 (segment (start 131.1 121.3612) (end 126.658 116.9192) (width 0.25) (layer F.Cu) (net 9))
 (segment (start 126.658 116.9192) (end 123.1387 116.9192) (width 0.25) (layer F.Cu) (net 9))
 (segment (start 123.1387 116.9192) (end 121.3131 118.7448) (width 0.25) (layer F.Cu) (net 9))
 (segment (start 121.3131 118.7448) (end 120.1548 118.7448) (width 0.25) (layer F.Cu) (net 9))
 (segment (start 120.1548 118.7448) (end 120.02 118.61) (width 0.25) (layer F.Cu) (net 9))
 (segment (start 131.9 121.6247) (end 131.9 121.5243) (width 0.25) (layer F.Cu) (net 10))
 (segment (start 131.9 121.5243) (end 126.7932 116.4175) (width 0.25) (layer F.Cu) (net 10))
 (segment (start 126.7932 116.4175) (end 118.7225 116.4175) (width 0.25) (layer F.Cu) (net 10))
 (segment (start 118.7225 116.4175) (end 117.17 117.97) (width 0.25) (layer F.Cu) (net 10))
 (segment (start 131.9 122.75) (end 131.9 121.6247) (width 0.25) (layer F.Cu) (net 10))
 (segment (start 132.7 131.25) (end 132.7 132.3753) (width 0.25) (layer F.Cu) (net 11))
 (segment (start 132.7 132.3753) (end 129.0695 132.3753) (width 0.25) (layer F.Cu) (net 11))
 (segment (start 129.0695 132.3753) (end 124.92 128.2258) (width 0.25) (layer F.Cu) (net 11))
 (segment (start 124.92 128.2258) (end 124.92 127.82) (width 0.25) (layer F.Cu) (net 11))
 (segment (start 162.46 99.72) (end 161.7114 99.72) (width 0.25) (layer F.Cu) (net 12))
 (segment (start 161.7114 99.72) (end 147.053 114.3784) (width 0.25) (layer F.Cu) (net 12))
 (segment (start 147.053 114.3784) (end 147.053 127.4589) (width 0.25) (layer F.Cu) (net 12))
 (segment (start 147.053 127.4589) (end 141.6862 132.8257) (width 0.25) (layer F.Cu) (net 12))
 (segment (start 141.6862 132.8257) (end 133.9504 132.8257) (width 0.25) (layer F.Cu) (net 12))
 (segment (start 133.9504 132.8257) (end 133.5 132.3753) (width 0.25) (layer F.Cu) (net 12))
 (segment (start 133.5 131.25) (end 133.5 132.3753) (width 0.25) (layer F.Cu) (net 12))
 (segment (start 162.46 76.2) (end 161.7114 76.2) (width 0.25) (layer F.Cu) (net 13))
 (segment (start 161.7114 76.2) (end 146.5453 91.3661) (width 0.25) (layer F.Cu) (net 13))
 (segment (start 146.5453 91.3661) (end 146.5453 127.3221) (width 0.25) (layer F.Cu) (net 13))
 (segment (start 146.5453 127.3221) (end 141.4921 132.3753) (width 0.25) (layer F.Cu) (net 13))
 (segment (start 141.4921 132.3753) (end 134.3 132.3753) (width 0.25) (layer F.Cu) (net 13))
 (segment (start 134.3 131.25) (end 134.3 132.3753) (width 0.25) (layer F.Cu) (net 13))
 (segment (start 135.1 131.25) (end 136.876 131.25) (width 0.25) (layer F.Cu) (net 14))
 (segment (start 136.876 131.25) (end 142.26 125.866) (width 0.25) (layer F.Cu) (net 14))
 (segment (start 142.26 125.866) (end 142.26 99.72) (width 0.25) (layer F.Cu) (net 14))
 (segment (start 137.6753 129.8) (end 138.5827 128.8926) (width 0.25) (layer F.Cu) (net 15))
 (segment (start 138.5827 128.8926) (end 138.5827 110.7166) (width 0.25) (layer F.Cu) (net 15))
 (segment (start 138.5827 110.7166) (end 137.3865 109.5204) (width 0.25) (layer F.Cu) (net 15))
 (segment (start 137.3865 109.5204) (end 137.3865 87.0113) (width 0.25) (layer F.Cu) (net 15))
 (segment (start 137.3865 87.0113) (end 142.24 82.1578) (width 0.25) (layer F.Cu) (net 15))
 (segment (start 142.24 82.1578) (end 142.24 76.2) (width 0.25) (layer F.Cu) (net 15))
 (segment (start 136.55 129.8) (end 137.6753 129.8) (width 0.25) (layer F.Cu) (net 15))
 (segment (start 136.55 129) (end 137.6753 129) (width 0.25) (layer F.Cu) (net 16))
 (segment (start 127.5726 101.7225) (end 124.0625 101.7225) (width 0.25) (layer B.Cu) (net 16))
 (segment (start 124.0625 101.7225) (end 122.06 99.72) (width 0.25) (layer B.Cu) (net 16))
 (segment (start 137.6753 129) (end 138.1324 128.5429) (width 0.25) (layer F.Cu) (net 16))
 (segment (start 138.1324 128.5429) (end 138.1324 112.2823) (width 0.25) (layer F.Cu) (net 16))
 (segment (start 138.1324 112.2823) (end 127.5726 101.7225) (width 0.25) (layer F.Cu) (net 16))
 (via (at 127.5726 101.7225) (size 0.8) (layers F.Cu B.Cu) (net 16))
 (segment (start 122.06 76.2) (end 122.06 97.2356) (width 0.25) (layer F.Cu) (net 17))
 (segment (start 122.06 97.2356) (end 137.6753 112.8509) (width 0.25) (layer F.Cu) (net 17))
 (segment (start 137.6753 112.8509) (end 137.6753 128.2) (width 0.25) (layer F.Cu) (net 17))
 (segment (start 136.55 128.2) (end 137.6753 128.2) (width 0.25) (layer F.Cu) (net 17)))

